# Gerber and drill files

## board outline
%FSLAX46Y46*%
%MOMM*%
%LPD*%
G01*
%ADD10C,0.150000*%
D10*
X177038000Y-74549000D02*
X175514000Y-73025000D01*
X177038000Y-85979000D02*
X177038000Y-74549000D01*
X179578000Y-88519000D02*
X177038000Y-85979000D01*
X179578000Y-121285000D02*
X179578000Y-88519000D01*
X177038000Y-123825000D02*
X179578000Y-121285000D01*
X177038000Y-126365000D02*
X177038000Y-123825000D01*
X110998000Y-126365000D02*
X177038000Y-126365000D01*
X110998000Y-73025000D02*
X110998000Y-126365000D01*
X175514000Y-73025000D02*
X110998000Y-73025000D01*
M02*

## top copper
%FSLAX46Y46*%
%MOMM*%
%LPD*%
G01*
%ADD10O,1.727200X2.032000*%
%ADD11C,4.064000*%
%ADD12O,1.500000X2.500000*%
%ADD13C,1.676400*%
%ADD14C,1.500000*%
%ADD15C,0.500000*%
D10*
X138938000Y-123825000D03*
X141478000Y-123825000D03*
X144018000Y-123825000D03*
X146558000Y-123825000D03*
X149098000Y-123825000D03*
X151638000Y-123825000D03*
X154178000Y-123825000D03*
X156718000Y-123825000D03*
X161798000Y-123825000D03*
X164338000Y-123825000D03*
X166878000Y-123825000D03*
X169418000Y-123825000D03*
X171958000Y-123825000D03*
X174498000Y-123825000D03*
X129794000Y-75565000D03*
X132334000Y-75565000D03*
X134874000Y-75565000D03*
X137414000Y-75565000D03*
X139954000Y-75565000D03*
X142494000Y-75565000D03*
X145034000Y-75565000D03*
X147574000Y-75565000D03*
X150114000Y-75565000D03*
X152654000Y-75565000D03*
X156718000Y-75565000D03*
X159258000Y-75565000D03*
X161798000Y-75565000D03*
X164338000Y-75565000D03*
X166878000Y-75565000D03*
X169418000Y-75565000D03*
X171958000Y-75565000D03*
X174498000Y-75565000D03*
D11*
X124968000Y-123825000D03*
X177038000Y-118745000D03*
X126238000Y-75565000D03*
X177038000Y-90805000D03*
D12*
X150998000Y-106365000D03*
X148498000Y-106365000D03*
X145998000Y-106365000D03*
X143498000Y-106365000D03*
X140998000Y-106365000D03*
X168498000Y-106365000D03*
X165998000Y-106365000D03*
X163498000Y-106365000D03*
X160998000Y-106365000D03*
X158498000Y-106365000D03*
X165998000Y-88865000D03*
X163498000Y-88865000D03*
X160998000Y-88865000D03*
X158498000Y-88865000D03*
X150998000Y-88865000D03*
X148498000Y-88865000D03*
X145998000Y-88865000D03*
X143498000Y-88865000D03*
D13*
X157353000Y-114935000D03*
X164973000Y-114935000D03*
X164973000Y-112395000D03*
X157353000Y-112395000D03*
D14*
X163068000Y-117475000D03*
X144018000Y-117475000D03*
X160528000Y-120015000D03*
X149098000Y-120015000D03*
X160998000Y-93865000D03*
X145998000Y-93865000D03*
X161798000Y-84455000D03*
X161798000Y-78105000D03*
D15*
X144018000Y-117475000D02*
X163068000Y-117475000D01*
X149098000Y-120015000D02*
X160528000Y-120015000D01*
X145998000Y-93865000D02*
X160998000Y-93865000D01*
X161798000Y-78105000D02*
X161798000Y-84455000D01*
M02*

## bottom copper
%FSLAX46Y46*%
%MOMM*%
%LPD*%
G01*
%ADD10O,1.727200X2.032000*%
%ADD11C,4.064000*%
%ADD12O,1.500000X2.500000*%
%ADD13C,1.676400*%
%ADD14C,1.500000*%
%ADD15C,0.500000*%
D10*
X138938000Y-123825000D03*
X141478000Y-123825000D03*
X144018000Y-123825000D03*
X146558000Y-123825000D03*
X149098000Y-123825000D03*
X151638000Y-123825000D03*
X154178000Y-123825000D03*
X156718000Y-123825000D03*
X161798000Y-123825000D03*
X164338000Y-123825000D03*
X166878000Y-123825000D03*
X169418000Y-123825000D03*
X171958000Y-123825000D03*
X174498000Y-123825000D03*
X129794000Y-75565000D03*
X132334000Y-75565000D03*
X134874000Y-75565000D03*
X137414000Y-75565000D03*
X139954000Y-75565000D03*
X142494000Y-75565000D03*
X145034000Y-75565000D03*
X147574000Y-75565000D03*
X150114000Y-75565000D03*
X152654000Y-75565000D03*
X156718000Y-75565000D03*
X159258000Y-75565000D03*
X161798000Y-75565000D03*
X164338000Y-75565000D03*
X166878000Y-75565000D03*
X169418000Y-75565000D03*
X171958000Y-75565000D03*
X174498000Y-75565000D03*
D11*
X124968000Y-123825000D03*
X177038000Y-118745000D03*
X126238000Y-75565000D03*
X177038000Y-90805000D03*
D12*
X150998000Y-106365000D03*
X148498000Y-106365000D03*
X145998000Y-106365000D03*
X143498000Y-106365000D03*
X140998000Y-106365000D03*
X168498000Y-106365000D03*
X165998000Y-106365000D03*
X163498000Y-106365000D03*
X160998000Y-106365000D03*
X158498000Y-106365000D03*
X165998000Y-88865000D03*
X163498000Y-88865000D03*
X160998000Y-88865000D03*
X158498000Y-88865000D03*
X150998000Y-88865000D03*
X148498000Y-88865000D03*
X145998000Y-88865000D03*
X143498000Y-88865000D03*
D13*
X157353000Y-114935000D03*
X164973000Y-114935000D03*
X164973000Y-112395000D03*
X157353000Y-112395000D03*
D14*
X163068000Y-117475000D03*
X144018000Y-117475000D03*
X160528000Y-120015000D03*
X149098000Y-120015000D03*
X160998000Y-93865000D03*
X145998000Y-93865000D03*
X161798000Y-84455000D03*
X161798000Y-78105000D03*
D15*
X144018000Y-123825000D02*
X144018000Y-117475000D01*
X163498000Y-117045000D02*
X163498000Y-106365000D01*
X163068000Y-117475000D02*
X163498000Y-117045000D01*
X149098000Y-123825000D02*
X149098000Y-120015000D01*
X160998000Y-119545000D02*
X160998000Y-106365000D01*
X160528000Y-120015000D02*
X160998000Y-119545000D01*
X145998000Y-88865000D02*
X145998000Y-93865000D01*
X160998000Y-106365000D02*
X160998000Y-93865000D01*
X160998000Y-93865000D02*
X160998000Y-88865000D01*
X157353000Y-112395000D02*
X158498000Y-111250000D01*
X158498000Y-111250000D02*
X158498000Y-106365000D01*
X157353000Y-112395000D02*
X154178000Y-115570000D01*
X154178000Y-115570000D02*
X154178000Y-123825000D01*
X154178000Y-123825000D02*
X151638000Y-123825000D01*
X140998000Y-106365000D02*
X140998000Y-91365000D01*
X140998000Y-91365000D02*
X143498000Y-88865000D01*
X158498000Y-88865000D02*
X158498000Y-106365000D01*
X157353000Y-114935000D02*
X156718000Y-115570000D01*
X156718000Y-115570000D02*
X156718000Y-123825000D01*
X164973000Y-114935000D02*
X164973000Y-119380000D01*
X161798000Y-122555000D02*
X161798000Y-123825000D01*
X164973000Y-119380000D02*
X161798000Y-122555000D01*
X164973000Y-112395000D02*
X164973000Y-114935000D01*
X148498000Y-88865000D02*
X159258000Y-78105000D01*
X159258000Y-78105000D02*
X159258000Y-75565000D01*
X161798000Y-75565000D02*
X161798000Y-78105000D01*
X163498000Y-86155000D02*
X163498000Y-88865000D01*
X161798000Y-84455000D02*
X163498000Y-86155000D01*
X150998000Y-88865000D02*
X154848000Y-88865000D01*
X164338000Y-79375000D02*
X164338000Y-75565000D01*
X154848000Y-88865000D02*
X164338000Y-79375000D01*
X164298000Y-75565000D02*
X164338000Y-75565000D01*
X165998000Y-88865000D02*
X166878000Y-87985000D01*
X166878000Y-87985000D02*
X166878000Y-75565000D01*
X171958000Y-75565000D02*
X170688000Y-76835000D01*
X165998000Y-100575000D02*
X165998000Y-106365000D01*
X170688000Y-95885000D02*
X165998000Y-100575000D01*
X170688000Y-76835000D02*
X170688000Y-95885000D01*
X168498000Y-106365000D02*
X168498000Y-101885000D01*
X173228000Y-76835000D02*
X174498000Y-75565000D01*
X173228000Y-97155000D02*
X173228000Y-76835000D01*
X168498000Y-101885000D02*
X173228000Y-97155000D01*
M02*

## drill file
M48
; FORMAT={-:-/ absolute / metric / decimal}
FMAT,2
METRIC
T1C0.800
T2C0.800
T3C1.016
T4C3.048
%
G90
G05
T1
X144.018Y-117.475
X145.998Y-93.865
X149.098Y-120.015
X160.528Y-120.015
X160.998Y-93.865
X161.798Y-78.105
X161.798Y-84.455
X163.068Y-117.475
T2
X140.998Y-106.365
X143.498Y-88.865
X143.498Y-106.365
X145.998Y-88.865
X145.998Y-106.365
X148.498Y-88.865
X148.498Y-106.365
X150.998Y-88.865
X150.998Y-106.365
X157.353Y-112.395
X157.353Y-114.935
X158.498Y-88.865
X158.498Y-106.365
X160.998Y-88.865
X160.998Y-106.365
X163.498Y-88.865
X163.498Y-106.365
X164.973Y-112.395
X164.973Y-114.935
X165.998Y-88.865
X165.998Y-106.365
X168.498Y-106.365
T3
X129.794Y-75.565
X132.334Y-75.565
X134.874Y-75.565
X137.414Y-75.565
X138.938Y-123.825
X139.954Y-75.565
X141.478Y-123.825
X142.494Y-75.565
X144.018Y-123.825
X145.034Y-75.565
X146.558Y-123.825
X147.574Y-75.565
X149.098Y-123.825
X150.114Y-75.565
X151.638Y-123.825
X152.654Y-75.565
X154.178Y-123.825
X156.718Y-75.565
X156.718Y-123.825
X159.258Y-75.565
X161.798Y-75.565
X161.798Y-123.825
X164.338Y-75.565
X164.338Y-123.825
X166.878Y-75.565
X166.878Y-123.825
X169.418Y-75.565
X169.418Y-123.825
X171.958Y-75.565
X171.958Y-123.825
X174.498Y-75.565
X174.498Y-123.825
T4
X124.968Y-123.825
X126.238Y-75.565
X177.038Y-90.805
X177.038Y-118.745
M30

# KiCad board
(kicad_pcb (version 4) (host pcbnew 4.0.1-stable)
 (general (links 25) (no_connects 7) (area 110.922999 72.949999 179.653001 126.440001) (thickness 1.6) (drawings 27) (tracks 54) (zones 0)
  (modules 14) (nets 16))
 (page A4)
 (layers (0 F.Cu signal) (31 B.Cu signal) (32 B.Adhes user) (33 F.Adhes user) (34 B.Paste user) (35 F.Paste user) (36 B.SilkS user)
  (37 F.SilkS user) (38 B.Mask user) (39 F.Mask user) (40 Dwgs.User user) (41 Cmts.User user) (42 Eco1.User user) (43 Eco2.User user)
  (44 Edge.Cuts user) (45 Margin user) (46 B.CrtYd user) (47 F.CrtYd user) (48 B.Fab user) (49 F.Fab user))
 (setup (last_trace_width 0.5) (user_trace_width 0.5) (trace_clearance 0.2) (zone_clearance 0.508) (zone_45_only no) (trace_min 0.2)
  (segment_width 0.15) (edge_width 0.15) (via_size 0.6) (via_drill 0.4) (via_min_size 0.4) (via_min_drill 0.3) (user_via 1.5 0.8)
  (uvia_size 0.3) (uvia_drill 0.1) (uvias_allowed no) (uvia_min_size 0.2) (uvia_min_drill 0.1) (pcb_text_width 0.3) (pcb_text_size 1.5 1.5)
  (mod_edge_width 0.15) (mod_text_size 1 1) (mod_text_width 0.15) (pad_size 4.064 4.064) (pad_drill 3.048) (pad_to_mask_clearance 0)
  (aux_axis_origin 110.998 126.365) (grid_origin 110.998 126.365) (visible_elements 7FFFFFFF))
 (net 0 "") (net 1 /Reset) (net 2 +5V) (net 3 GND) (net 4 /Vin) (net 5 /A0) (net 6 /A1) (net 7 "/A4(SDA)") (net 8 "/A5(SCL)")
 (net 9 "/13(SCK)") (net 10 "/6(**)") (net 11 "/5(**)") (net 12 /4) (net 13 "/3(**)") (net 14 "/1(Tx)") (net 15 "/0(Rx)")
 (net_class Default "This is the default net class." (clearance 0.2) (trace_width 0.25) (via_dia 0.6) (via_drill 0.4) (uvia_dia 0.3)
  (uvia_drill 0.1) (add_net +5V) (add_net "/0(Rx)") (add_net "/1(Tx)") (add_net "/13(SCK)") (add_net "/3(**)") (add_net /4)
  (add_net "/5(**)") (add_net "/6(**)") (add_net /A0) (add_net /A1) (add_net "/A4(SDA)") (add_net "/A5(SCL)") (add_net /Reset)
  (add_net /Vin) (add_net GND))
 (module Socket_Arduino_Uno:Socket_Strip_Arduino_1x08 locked (layer F.Cu) (at 138.938 123.825)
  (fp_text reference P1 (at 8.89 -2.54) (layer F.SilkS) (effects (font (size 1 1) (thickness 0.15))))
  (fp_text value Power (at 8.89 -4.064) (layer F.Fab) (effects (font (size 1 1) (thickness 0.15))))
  (pad 1 thru_hole oval (at 0 0) (size 1.7272 2.032) (drill 1.016) (layers *.Cu *.Mask F.SilkS))
  (pad 2 thru_hole oval (at 2.54 0) (size 1.7272 2.032) (drill 1.016) (layers *.Cu *.Mask F.SilkS))
  (pad 3 thru_hole oval (at 5.08 0) (size 1.7272 2.032) (drill 1.016) (layers *.Cu *.Mask F.SilkS) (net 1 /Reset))
  (pad 4 thru_hole oval (at 7.62 0) (size 1.7272 2.032) (drill 1.016) (layers *.Cu *.Mask F.SilkS))
  (pad 5 thru_hole oval (at 10.16 0) (size 1.7272 2.032) (drill 1.016) (layers *.Cu *.Mask F.SilkS) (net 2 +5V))
  (pad 6 thru_hole oval (at 12.7 0) (size 1.7272 2.032) (drill 1.016) (layers *.Cu *.Mask F.SilkS) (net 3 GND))
  (pad 7 thru_hole oval (at 15.24 0) (size 1.7272 2.032) (drill 1.016) (layers *.Cu *.Mask F.SilkS) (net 3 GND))
  (pad 8 thru_hole oval (at 17.78 0) (size 1.7272 2.032) (drill 1.016) (layers *.Cu *.Mask F.SilkS) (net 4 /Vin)))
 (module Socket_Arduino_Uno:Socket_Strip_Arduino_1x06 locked (layer F.Cu) (at 161.798 123.825)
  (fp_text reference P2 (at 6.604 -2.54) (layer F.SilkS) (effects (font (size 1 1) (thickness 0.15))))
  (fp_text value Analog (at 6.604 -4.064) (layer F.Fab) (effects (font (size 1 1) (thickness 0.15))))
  (pad 1 thru_hole oval (at 0 0) (size 1.7272 2.032) (drill 1.016) (layers *.Cu *.Mask F.SilkS) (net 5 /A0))
  (pad 2 thru_hole oval (at 2.54 0) (size 1.7272 2.032) (drill 1.016) (layers *.Cu *.Mask F.SilkS) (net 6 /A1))
  (pad 3 thru_hole oval (at 5.08 0) (size 1.7272 2.032) (drill 1.016) (layers *.Cu *.Mask F.SilkS))
  (pad 4 thru_hole oval (at 7.62 0) (size 1.7272 2.032) (drill 1.016) (layers *.Cu *.Mask F.SilkS))
  (pad 5 thru_hole oval (at 10.16 0) (size 1.7272 2.032) (drill 1.016) (layers *.Cu *.Mask F.SilkS) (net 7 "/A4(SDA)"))
  (pad 6 thru_hole oval (at 12.7 0) (size 1.7272 2.032) (drill 1.016) (layers *.Cu *.Mask F.SilkS) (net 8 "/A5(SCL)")))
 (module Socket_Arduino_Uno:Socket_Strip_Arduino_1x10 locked (layer F.Cu) (at 129.794 75.565)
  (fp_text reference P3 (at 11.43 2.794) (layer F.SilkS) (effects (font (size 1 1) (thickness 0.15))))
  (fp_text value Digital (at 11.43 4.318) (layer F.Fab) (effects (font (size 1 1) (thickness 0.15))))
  (pad 1 thru_hole oval (at 0 0) (size 1.7272 2.032) (drill 1.016) (layers *.Cu *.Mask F.SilkS) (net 8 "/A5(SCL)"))
  (pad 2 thru_hole oval (at 2.54 0) (size 1.7272 2.032) (drill 1.016) (layers *.Cu *.Mask F.SilkS) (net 7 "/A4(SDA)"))
  (pad 3 thru_hole oval (at 5.08 0) (size 1.7272 2.032) (drill 1.016) (layers *.Cu *.Mask F.SilkS))
  (pad 4 thru_hole oval (at 7.62 0) (size 1.7272 2.032) (drill 1.016) (layers *.Cu *.Mask F.SilkS) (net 3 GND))
  (pad 5 thru_hole oval (at 10.16 0) (size 1.7272 2.032) (drill 1.016) (layers *.Cu *.Mask F.SilkS) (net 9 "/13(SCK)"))
  (pad 6 thru_hole oval (at 12.7 0) (size 1.7272 2.032) (drill 1.016) (layers *.Cu *.Mask F.SilkS))
  (pad 7 thru_hole oval (at 15.24 0) (size 1.7272 2.032) (drill 1.016) (layers *.Cu *.Mask F.SilkS))
  (pad 8 thru_hole oval (at 17.78 0) (size 1.7272 2.032) (drill 1.016) (layers *.Cu *.Mask F.SilkS))
  (pad 9 thru_hole oval (at 20.32 0) (size 1.7272 2.032) (drill 1.016) (layers *.Cu *.Mask F.SilkS))
  (pad 10 thru_hole oval (at 22.86 0) (size 1.7272 2.032) (drill 1.016) (layers *.Cu *.Mask F.SilkS)))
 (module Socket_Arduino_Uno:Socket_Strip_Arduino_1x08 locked (layer F.Cu) (at 156.718 75.565)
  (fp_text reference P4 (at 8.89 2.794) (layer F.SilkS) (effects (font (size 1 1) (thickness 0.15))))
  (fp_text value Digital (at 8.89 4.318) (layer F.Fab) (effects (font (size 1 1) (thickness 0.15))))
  (pad 1 thru_hole oval (at 0 0) (size 1.7272 2.032) (drill 1.016) (layers *.Cu *.Mask F.SilkS))
  (pad 2 thru_hole oval (at 2.54 0) (size 1.7272 2.032) (drill 1.016) (layers *.Cu *.Mask F.SilkS) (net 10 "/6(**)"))
  (pad 3 thru_hole oval (at 5.08 0) (size 1.7272 2.032) (drill 1.016) (layers *.Cu *.Mask F.SilkS) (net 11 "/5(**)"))
  (pad 4 thru_hole oval (at 7.62 0) (size 1.7272 2.032) (drill 1.016) (layers *.Cu *.Mask F.SilkS) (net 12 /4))
  (pad 5 thru_hole oval (at 10.16 0) (size 1.7272 2.032) (drill 1.016) (layers *.Cu *.Mask F.SilkS) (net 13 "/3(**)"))
  (pad 6 thru_hole oval (at 12.7 0) (size 1.7272 2.032) (drill 1.016) (layers *.Cu *.Mask F.SilkS))
  (pad 7 thru_hole oval (at 15.24 0) (size 1.7272 2.032) (drill 1.016) (layers *.Cu *.Mask F.SilkS) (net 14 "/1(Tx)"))
  (pad 8 thru_hole oval (at 17.78 0) (size 1.7272 2.032) (drill 1.016) (layers *.Cu *.Mask F.SilkS) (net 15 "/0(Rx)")))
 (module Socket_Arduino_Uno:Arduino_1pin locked (layer F.Cu) (at 124.968 123.825)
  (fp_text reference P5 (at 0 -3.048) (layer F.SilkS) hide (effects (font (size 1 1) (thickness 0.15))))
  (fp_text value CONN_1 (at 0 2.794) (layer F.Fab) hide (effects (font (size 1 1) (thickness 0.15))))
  (pad 1 thru_hole circle (at 0 0) (size 4.064 4.064) (drill 3.048) (layers *.Cu *.Mask F.SilkS)))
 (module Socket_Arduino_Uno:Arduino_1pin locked (layer F.Cu) (at 177.038 118.745)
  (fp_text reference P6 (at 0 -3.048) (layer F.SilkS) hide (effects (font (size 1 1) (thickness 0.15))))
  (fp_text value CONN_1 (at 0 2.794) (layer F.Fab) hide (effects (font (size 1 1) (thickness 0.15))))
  (pad 1 thru_hole circle (at 0 0) (size 4.064 4.064) (drill 3.048) (layers *.Cu *.Mask F.SilkS)))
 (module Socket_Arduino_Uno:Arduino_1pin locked (layer F.Cu) (at 126.238 75.565)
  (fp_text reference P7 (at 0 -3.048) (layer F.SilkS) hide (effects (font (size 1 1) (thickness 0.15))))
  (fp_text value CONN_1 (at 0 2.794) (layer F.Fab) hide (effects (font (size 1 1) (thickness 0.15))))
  (pad 1 thru_hole circle (at 0 0) (size 4.064 4.064) (drill 3.048) (layers *.Cu *.Mask F.SilkS)))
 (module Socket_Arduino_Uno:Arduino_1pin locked (layer F.Cu) (at 177.038 90.805)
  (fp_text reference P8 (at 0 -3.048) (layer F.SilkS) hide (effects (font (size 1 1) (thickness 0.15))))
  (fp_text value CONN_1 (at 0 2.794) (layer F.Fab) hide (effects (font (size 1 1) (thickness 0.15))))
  (pad 1 thru_hole circle (at 0 0) (size 4.064 4.064) (drill 3.048) (layers *.Cu *.Mask F.SilkS)))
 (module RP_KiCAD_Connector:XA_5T (layer F.Cu) (at 150.998 106.365 180)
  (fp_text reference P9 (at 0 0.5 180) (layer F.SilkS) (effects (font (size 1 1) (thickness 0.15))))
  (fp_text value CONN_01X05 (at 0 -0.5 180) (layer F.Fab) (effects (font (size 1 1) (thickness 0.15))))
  (pad 5 thru_hole oval (at 0 0 180) (size 1.5 2.5) (drill 0.8) (layers *.Cu *.Mask F.SilkS) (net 9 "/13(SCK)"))
  (pad 4 thru_hole oval (at 2.5 0 180) (size 1.5 2.5) (drill 0.8) (layers *.Cu *.Mask F.SilkS) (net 6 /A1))
  (pad 3 thru_hole oval (at 5 0 180) (size 1.5 2.5) (drill 0.8) (layers *.Cu *.Mask F.SilkS))
  (pad 2 thru_hole oval (at 7.5 0 180) (size 1.5 2.5) (drill 0.8) (layers *.Cu *.Mask F.SilkS) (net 4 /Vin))
  (pad 1 thru_hole oval (at 10 0 180) (size 1.5 2.5) (drill 0.8) (layers *.Cu *.Mask F.SilkS) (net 3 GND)))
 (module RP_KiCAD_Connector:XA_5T (layer F.Cu) (at 168.498 106.365 180)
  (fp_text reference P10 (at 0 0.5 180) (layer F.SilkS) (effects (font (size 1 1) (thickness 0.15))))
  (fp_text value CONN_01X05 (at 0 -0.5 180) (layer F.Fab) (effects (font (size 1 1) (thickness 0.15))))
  (pad 5 thru_hole oval (at 0 0 180) (size 1.5 2.5) (drill 0.8) (layers *.Cu *.Mask F.SilkS) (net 15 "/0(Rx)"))
  (pad 4 thru_hole oval (at 2.5 0 180) (size 1.5 2.5) (drill 0.8) (layers *.Cu *.Mask F.SilkS) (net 14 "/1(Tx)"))
  (pad 3 thru_hole oval (at 5 0 180) (size 1.5 2.5) (drill 0.8) (layers *.Cu *.Mask F.SilkS) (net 1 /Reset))
  (pad 2 thru_hole oval (at 7.5 0 180) (size 1.5 2.5) (drill 0.8) (layers *.Cu *.Mask F.SilkS) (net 2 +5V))
  (pad 1 thru_hole oval (at 10 0 180) (size 1.5 2.5) (drill 0.8) (layers *.Cu *.Mask F.SilkS) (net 3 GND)))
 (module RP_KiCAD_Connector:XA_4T (layer F.Cu) (at 165.998 88.865 180)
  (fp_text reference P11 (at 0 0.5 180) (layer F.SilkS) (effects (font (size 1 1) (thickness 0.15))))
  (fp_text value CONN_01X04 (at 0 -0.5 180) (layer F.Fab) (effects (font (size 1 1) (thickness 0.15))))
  (pad 4 thru_hole oval (at 0 0 180) (size 1.5 2.5) (drill 0.8) (layers *.Cu *.Mask F.SilkS) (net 13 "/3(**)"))
  (pad 3 thru_hole oval (at 2.5 0 180) (size 1.5 2.5) (drill 0.8) (layers *.Cu *.Mask F.SilkS) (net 11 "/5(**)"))
  (pad 2 thru_hole oval (at 5 0 180) (size 1.5 2.5) (drill 0.8) (layers *.Cu *.Mask F.SilkS) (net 2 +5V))
  (pad 1 thru_hole oval (at 7.5 0 180) (size 1.5 2.5) (drill 0.8) (layers *.Cu *.Mask F.SilkS) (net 3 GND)))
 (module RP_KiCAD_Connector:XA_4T (layer F.Cu) (at 150.998 88.865 180)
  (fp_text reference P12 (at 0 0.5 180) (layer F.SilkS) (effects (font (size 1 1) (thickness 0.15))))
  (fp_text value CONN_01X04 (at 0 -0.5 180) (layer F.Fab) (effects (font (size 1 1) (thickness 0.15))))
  (pad 4 thru_hole oval (at 0 0 180) (size 1.5 2.5) (drill 0.8) (layers *.Cu *.Mask F.SilkS) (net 12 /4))
  (pad 3 thru_hole oval (at 2.5 0 180) (size 1.5 2.5) (drill 0.8) (layers *.Cu *.Mask F.SilkS) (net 10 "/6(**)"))
  (pad 2 thru_hole oval (at 5 0 180) (size 1.5 2.5) (drill 0.8) (layers *.Cu *.Mask F.SilkS) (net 2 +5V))
  (pad 1 thru_hole oval (at 7.5 0 180) (size 1.5 2.5) (drill 0.8) (layers *.Cu *.Mask F.SilkS) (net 3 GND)))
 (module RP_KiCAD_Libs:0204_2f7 (layer F.Cu) (at 161.163 114.935)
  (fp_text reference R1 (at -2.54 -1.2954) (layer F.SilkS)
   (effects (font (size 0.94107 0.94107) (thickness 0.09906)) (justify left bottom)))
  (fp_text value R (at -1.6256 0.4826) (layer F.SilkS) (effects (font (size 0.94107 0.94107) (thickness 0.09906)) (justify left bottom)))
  (pad 1 thru_hole circle (at -3.81 0) (size 1.6764 1.6764) (drill 0.8) (layers *.Cu *.Mask) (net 4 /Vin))
  (pad 2 thru_hole circle (at 3.81 0) (size 1.6764 1.6764) (drill 0.8) (layers *.Cu *.Mask) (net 5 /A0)))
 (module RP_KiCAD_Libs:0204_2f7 (layer F.Cu) (at 161.163 112.395 180)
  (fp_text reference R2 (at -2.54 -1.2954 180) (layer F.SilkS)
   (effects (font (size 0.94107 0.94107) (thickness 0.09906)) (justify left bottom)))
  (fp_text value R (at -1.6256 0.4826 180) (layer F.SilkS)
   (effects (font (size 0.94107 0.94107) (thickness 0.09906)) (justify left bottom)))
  (pad 1 thru_hole circle (at -3.81 0 180) (size 1.6764 1.6764) (drill 0.8) (layers *.Cu *.Mask) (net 5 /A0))
  (pad 2 thru_hole circle (at 3.81 0 180) (size 1.6764 1.6764) (drill 0.8) (layers *.Cu *.Mask) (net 3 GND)))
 (gr_line (start 177.038 74.549) (end 175.514 73.025) (angle 90) (layer Edge.Cuts) (width 0.15))
 (gr_line (start 177.038 85.979) (end 177.038 74.549) (angle 90) (layer Edge.Cuts) (width 0.15))
 (gr_line (start 179.578 88.519) (end 177.038 85.979) (angle 90) (layer Edge.Cuts) (width 0.15))
 (gr_line (start 179.578 121.285) (end 179.578 88.519) (angle 90) (layer Edge.Cuts) (width 0.15))
 (gr_line (start 177.038 123.825) (end 179.578 121.285) (angle 90) (layer Edge.Cuts) (width 0.15))
 (gr_line (start 177.038 126.365) (end 177.038 123.825) (angle 90) (layer Edge.Cuts) (width 0.15))
 (gr_line (start 110.998 126.365) (end 177.038 126.365) (angle 90) (layer Edge.Cuts) (width 0.15))
 (gr_line (start 110.998 73.025) (end 110.998 126.365) (angle 90) (layer Edge.Cuts) (width 0.15))
 (gr_line (start 175.514 73.025) (end 110.998 73.025) (angle 90) (layer Edge.Cuts) (width 0.15))
 (segment (start 144.018 123.825) (end 144.018 117.475) (width 0.5) (layer B.Cu) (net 1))
 (segment (start 163.498 117.045) (end 163.498 106.365) (width 0.5) (layer B.Cu) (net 1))
 (segment (start 163.068 117.475) (end 163.498 117.045) (width 0.5) (layer B.Cu) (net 1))
 (via (at 163.068 117.475) (size 1.5) (drill 0.8) (layers F.Cu B.Cu) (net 1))
 (segment (start 144.018 117.475) (end 163.068 117.475) (width 0.5) (layer F.Cu) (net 1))
 (via (at 144.018 117.475) (size 1.5) (drill 0.8) (layers F.Cu B.Cu) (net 1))
 (segment (start 149.098 123.825) (end 149.098 120.015) (width 0.5) (layer B.Cu) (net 2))
 (segment (start 160.998 119.545) (end 160.998 106.365) (width 0.5) (layer B.Cu) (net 2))
 (segment (start 160.528 120.015) (end 160.998 119.545) (width 0.5) (layer B.Cu) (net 2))
 (via (at 160.528 120.015) (size 1.5) (drill 0.8) (layers F.Cu B.Cu) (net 2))
 (segment (start 149.098 120.015) (end 160.528 120.015) (width 0.5) (layer F.Cu) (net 2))
 (via (at 149.098 120.015) (size 1.5) (drill 0.8) (layers F.Cu B.Cu) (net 2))
 (segment (start 145.998 88.865) (end 145.998 93.865) (width 0.5) (layer B.Cu) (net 2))
 (via (at 160.998 93.865) (size 1.5) (drill 0.8) (layers F.Cu B.Cu) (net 2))
 (segment (start 145.998 93.865) (end 160.998 93.865) (width 0.5) (layer F.Cu) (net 2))
 (via (at 145.998 93.865) (size 1.5) (drill 0.8) (layers F.Cu B.Cu) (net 2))
 (segment (start 160.998 106.365) (end 160.998 93.865) (width 0.5) (layer B.Cu) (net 2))
 (segment (start 160.998 93.865) (end 160.998 88.865) (width 0.5) (layer B.Cu) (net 2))
 (segment (start 157.353 112.395) (end 158.498 111.25) (width 0.5) (layer B.Cu) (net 3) (status 400000))
 (segment (start 158.498 111.25) (end 158.498 106.365) (width 0.5) (layer B.Cu) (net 3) (status 800000))
 (segment (start 157.353 112.395) (end 154.178 115.57) (width 0.5) (layer B.Cu) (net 3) (status 400000))
 (segment (start 154.178 115.57) (end 154.178 123.825) (width 0.5) (layer B.Cu) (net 3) (status 800000))
 (segment (start 154.178 123.825) (end 151.638 123.825) (width 0.5) (layer B.Cu) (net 3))
 (segment (start 140.998 106.365) (end 140.998 91.365) (width 0.5) (layer B.Cu) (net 3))
 (segment (start 140.998 91.365) (end 143.498 88.865) (width 0.5) (layer B.Cu) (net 3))
 (segment (start 158.498 88.865) (end 158.498 106.365) (width 0.5) (layer B.Cu) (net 3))
 (segment (start 157.353 114.935) (end 156.718 115.57) (width 0.5) (layer B.Cu) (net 4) (status 400000))
 (segment (start 156.718 115.57) (end 156.718 123.825) (width 0.5) (layer B.Cu) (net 4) (status 800000))
 (segment (start 164.973 114.935) (end 164.973 119.38) (width 0.5) (layer B.Cu) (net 5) (status 400000))
 (segment (start 161.798 122.555) (end 161.798 123.825) (width 0.5) (layer B.Cu) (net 5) (status 800000))
 (segment (start 164.973 119.38) (end 161.798 122.555) (width 0.5) (layer B.Cu) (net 5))
 (segment (start 164.973 112.395) (end 164.973 114.935) (width 0.5) (layer B.Cu) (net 5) (status C00000))
 (segment (start 148.498 88.865) (end 159.258 78.105) (width 0.5) (layer B.Cu) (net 10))
 (segment (start 159.258 78.105) (end 159.258 75.565) (width 0.5) (layer B.Cu) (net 10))
 (segment (start 161.798 75.565) (end 161.798 78.105) (width 0.5) (layer B.Cu) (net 11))
 (segment (start 163.498 86.155) (end 163.498 88.865) (width 0.5) (layer B.Cu) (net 11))
 (segment (start 161.798 84.455) (end 163.498 86.155) (width 0.5) (layer B.Cu) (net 11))
 (via (at 161.798 84.455) (size 1.5) (drill 0.8) (layers F.Cu B.Cu) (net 11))
 (segment (start 161.798 78.105) (end 161.798 84.455) (width 0.5) (layer F.Cu) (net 11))
 (via (at 161.798 78.105) (size 1.5) (drill 0.8) (layers F.Cu B.Cu) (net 11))
 (segment (start 150.998 88.865) (end 154.848 88.865) (width 0.5) (layer B.Cu) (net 12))
 (segment (start 164.338 79.375) (end 164.338 75.565) (width 0.5) (layer B.Cu) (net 12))
 (segment (start 154.848 88.865) (end 164.338 79.375) (width 0.5) (layer B.Cu) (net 12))
 (segment (start 164.298 75.565) (end 164.338 75.565) (width 0.5) (layer B.Cu) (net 12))
 (segment (start 165.998 88.865) (end 166.878 87.985) (width 0.5) (layer B.Cu) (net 13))
 (segment (start 166.878 87.985) (end 166.878 75.565) (width 0.5) (layer B.Cu) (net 13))
 (segment (start 171.958 75.565) (end 170.688 76.835) (width 0.5) (layer B.Cu) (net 14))
 (segment (start 165.998 100.575) (end 165.998 106.365) (width 0.5) (layer B.Cu) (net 14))
 (segment (start 170.688 95.885) (end 165.998 100.575) (width 0.5) (layer B.Cu) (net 14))
 (segment (start 170.688 76.835) (end 170.688 95.885) (width 0.5) (layer B.Cu) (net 14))
 (segment (start 168.498 106.365) (end 168.498 101.885) (width 0.5) (layer B.Cu) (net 15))
 (segment (start 173.228 76.835) (end 174.498 75.565) (width 0.5) (layer B.Cu) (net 15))
 (segment (start 173.228 97.155) (end 173.228 76.835) (width 0.5) (layer B.Cu) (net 15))
 (segment (start 168.498 101.885) (end 173.228 97.155) (width 0.5) (layer B.Cu) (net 15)))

